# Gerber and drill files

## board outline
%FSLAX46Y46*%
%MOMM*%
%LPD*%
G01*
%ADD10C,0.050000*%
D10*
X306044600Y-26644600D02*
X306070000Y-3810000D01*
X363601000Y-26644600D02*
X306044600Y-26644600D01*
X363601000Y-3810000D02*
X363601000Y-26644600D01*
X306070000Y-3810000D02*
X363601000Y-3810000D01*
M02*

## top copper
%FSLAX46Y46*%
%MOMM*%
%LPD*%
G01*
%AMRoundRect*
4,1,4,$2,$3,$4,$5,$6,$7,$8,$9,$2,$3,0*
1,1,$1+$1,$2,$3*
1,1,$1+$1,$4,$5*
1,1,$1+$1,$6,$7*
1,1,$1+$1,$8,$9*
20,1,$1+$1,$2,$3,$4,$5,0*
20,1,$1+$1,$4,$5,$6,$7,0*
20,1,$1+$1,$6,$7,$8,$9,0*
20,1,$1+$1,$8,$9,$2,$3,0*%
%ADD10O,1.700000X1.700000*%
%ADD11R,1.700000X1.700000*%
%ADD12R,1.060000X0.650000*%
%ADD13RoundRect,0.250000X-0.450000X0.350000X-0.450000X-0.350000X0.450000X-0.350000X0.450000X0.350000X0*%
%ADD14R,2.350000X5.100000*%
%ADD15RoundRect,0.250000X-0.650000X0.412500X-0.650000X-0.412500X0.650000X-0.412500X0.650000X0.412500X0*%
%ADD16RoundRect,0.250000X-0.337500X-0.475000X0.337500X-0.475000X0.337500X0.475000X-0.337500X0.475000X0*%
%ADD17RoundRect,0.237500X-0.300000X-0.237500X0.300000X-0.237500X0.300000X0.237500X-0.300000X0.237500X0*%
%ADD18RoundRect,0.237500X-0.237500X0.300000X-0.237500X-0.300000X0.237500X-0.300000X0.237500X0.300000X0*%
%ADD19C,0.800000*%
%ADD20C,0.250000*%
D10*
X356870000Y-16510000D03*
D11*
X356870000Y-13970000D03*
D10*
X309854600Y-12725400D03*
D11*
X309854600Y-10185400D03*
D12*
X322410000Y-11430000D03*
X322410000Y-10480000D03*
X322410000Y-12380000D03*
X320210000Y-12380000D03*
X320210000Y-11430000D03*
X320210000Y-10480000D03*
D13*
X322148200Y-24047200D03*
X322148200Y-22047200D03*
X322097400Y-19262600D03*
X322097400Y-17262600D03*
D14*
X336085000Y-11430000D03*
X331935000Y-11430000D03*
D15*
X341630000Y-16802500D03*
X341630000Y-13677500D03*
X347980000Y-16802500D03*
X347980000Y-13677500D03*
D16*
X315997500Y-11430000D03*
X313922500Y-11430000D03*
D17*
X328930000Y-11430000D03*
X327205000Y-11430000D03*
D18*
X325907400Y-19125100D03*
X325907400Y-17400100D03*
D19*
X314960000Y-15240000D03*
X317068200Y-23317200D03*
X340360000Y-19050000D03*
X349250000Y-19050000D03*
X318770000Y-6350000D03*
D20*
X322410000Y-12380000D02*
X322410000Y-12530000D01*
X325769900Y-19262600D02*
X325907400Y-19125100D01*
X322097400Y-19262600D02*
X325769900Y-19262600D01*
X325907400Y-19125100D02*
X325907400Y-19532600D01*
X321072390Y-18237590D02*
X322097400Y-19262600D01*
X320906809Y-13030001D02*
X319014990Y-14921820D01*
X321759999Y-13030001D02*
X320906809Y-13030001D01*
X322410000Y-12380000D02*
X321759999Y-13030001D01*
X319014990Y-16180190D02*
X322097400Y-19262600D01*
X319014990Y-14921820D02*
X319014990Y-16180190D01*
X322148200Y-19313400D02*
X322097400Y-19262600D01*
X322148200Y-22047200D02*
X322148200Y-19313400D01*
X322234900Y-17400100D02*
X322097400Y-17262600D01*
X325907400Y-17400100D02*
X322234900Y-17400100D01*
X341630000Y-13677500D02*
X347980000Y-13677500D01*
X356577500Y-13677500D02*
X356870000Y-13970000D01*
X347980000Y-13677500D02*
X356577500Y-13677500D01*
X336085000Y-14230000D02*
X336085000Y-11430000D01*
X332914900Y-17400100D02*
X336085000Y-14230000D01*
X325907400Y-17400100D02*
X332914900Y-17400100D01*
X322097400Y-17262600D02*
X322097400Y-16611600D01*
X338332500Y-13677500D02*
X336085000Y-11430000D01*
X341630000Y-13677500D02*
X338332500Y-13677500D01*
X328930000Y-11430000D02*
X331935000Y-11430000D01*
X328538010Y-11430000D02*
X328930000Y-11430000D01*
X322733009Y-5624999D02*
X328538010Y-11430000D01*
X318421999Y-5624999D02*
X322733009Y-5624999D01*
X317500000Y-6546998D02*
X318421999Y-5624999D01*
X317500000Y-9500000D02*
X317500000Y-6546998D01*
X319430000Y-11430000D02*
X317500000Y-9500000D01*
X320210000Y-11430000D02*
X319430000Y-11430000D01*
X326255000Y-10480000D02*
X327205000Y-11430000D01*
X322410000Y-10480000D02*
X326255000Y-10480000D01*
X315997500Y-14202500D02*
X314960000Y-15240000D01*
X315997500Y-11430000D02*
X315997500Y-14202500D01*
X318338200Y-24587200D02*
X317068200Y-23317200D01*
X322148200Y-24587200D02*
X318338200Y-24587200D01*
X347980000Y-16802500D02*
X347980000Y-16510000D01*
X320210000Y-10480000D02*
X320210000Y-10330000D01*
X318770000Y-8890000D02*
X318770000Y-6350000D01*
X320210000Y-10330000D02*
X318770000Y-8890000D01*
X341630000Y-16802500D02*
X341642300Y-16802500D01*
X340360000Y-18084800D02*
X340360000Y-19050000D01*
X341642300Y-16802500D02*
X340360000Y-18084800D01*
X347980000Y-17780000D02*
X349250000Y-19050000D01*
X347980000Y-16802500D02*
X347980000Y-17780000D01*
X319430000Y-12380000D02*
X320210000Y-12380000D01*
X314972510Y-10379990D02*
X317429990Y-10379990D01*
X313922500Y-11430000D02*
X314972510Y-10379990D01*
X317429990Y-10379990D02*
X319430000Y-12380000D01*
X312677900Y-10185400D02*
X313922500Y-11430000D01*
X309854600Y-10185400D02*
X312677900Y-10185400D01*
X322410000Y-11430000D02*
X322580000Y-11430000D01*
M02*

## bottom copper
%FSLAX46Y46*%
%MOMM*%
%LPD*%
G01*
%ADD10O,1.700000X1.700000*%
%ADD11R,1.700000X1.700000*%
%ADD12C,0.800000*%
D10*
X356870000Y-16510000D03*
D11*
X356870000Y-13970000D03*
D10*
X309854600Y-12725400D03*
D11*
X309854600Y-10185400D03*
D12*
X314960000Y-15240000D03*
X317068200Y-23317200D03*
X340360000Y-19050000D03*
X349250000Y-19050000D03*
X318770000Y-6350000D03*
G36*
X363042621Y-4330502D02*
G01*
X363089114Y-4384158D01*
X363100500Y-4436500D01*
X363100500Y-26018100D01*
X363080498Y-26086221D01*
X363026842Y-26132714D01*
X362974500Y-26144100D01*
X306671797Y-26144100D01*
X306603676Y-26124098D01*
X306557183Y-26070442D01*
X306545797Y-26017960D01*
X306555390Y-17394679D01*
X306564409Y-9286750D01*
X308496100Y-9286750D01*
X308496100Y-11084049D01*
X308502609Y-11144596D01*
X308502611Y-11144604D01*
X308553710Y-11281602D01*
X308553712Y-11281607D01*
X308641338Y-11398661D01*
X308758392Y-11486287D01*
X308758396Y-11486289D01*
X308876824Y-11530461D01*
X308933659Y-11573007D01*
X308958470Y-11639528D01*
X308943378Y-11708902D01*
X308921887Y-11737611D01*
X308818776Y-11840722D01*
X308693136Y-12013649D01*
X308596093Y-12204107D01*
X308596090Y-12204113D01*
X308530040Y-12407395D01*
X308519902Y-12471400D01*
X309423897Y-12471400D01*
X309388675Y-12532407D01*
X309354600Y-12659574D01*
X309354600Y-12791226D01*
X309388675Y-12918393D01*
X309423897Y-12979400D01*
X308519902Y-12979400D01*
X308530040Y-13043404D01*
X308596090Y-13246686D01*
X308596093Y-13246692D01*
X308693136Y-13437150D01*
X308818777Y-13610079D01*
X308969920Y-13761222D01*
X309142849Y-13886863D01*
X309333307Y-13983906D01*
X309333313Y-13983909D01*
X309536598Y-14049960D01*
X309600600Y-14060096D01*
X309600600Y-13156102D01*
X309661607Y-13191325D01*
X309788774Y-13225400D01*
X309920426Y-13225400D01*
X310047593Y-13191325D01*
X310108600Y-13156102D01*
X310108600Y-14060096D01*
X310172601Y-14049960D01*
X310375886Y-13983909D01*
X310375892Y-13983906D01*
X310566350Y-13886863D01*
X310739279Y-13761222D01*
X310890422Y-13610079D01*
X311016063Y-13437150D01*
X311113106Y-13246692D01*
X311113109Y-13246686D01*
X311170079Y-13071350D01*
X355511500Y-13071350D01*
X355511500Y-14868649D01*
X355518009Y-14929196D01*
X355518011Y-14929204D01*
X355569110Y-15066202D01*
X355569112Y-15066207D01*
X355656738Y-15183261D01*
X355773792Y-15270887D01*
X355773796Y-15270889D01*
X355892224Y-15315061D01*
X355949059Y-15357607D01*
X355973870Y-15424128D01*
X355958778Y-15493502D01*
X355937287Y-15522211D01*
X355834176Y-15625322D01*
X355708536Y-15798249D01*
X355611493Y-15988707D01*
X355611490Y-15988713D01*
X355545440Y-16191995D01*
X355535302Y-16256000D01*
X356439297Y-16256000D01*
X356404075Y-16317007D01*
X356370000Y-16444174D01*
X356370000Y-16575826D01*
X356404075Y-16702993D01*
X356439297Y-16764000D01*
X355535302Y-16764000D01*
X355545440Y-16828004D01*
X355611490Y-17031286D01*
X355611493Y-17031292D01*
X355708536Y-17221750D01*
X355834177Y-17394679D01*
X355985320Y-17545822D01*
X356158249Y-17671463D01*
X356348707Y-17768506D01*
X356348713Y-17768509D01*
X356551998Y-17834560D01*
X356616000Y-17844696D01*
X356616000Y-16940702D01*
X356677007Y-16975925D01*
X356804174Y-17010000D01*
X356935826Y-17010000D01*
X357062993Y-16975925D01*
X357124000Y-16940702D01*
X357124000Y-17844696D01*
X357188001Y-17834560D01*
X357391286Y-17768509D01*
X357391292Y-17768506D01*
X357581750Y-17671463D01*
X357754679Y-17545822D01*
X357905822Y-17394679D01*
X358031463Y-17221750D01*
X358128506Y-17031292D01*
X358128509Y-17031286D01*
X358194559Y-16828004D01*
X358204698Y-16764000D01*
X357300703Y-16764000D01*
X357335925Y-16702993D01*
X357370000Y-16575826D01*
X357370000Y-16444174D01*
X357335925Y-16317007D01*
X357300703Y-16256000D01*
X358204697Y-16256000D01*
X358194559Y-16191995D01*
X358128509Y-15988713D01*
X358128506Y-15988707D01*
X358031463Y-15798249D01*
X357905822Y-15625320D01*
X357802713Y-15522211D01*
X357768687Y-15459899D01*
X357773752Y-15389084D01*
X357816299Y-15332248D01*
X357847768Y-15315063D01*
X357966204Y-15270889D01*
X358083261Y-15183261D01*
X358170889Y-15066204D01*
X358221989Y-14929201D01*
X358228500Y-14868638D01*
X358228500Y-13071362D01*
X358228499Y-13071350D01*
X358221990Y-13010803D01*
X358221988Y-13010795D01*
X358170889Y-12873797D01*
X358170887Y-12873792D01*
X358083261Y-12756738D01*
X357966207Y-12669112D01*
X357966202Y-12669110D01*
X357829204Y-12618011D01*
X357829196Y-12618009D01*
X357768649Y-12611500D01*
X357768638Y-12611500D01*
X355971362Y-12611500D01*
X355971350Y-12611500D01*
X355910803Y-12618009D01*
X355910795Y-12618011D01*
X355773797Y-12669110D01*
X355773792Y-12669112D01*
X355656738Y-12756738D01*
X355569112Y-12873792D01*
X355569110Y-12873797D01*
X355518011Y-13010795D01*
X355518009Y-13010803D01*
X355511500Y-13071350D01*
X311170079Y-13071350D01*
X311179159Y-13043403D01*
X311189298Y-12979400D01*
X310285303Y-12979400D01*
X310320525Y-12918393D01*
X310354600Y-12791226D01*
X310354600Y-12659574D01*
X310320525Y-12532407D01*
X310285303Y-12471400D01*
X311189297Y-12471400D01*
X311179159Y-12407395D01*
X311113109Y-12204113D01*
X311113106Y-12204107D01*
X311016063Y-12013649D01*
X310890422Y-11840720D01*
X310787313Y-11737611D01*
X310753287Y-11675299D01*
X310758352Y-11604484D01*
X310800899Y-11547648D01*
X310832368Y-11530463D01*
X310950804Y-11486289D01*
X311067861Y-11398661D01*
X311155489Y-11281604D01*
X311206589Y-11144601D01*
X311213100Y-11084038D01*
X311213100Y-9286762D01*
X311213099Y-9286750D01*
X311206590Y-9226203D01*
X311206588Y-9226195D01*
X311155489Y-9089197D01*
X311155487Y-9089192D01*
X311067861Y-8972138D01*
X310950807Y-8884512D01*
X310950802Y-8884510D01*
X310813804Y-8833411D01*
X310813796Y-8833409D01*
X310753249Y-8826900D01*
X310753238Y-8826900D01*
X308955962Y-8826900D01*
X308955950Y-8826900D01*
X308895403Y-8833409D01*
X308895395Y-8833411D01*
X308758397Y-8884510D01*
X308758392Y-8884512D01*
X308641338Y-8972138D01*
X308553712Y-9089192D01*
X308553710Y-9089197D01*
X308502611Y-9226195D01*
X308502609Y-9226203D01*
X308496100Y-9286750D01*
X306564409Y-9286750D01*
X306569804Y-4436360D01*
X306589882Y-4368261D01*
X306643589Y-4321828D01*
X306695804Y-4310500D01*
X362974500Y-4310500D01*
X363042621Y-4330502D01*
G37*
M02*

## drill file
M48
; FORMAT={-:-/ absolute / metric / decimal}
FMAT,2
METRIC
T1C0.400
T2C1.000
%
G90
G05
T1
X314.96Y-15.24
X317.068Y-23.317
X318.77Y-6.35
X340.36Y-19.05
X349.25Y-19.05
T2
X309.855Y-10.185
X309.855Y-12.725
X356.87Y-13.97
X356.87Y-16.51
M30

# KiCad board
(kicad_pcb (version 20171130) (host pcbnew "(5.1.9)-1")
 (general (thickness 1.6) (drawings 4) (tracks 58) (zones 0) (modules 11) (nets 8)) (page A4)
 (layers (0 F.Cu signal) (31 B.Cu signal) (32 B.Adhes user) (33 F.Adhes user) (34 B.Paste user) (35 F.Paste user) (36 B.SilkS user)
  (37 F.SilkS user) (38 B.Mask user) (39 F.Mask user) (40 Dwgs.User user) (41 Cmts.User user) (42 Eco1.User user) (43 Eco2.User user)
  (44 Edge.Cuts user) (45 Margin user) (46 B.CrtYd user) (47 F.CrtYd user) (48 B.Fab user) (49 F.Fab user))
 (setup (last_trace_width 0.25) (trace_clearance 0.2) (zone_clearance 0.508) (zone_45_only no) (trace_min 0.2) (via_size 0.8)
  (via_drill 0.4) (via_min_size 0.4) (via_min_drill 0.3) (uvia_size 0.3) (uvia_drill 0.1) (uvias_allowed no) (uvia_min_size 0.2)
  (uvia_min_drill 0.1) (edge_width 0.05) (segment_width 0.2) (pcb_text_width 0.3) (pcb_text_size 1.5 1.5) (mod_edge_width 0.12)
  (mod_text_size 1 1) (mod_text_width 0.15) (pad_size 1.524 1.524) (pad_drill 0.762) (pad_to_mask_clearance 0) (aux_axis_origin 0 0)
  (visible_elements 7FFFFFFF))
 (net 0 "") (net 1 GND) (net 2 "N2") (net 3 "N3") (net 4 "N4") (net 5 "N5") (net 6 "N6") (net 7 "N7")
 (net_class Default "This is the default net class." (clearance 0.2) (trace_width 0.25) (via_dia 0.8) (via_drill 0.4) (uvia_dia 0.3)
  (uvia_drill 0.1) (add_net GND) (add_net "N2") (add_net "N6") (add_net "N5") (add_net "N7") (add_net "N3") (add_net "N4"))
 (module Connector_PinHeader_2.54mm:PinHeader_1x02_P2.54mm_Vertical (layer F.Cu) (at 356.87 13.97)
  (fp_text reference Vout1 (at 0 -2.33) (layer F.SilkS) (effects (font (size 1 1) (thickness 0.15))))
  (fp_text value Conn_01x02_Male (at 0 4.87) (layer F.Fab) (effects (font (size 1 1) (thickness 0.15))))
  (pad 2 thru_hole oval (at 0 2.54) (size 1.7 1.7) (drill 1) (layers *.Cu *.Mask) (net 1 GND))
  (pad 1 thru_hole rect (at 0 0) (size 1.7 1.7) (drill 1) (layers *.Cu *.Mask) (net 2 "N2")))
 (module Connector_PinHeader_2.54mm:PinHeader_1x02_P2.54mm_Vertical (layer F.Cu) (at 309.8546 10.1854)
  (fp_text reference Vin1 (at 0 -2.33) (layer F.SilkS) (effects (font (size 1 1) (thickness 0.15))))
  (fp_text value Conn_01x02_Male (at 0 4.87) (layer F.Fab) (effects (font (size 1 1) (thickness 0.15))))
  (pad 2 thru_hole oval (at 0 2.54) (size 1.7 1.7) (drill 1) (layers *.Cu *.Mask) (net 1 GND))
  (pad 1 thru_hole rect (at 0 0) (size 1.7 1.7) (drill 1) (layers *.Cu *.Mask) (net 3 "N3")))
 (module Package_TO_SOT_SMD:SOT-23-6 (layer F.Cu) (at 321.31 11.43)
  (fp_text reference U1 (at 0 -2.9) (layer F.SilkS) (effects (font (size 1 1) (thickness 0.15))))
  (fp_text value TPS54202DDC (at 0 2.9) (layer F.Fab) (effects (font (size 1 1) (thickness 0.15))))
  (pad 5 smd rect (at 1.1 0) (size 1.06 0.65) (layers F.Cu F.Paste F.Mask) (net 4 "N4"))
  (pad 6 smd rect (at 1.1 -0.95) (size 1.06 0.65) (layers F.Cu F.Paste F.Mask) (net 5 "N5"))
  (pad 4 smd rect (at 1.1 0.95) (size 1.06 0.65) (layers F.Cu F.Paste F.Mask) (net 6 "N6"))
  (pad 3 smd rect (at -1.1 0.95) (size 1.06 0.65) (layers F.Cu F.Paste F.Mask) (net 3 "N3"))
  (pad 2 smd rect (at -1.1 0) (size 1.06 0.65) (layers F.Cu F.Paste F.Mask) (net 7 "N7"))
  (pad 1 smd rect (at -1.1 -0.95) (size 1.06 0.65) (layers F.Cu F.Paste F.Mask) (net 1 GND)))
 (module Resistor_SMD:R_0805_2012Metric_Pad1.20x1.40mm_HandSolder (layer F.Cu) (at 322.1482 23.0472 270)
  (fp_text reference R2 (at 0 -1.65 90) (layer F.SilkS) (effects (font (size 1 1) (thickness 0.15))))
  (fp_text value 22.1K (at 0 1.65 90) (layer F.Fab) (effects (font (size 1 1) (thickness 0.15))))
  (pad 2 smd roundrect (at 1 0 270) (size 1.2 1.4) (layers F.Cu F.Paste F.Mask) (roundrect_rratio 0.208333) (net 1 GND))
  (pad 1 smd roundrect (at -1 0 270) (size 1.2 1.4) (layers F.Cu F.Paste F.Mask) (roundrect_rratio 0.208333) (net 6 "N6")))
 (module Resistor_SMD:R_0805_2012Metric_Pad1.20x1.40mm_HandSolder (layer F.Cu) (at 322.0974 18.2626 270)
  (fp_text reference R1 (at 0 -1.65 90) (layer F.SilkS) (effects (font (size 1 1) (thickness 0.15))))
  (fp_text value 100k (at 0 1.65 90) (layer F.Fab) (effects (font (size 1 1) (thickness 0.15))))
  (pad 2 smd roundrect (at 1 0 270) (size 1.2 1.4) (layers F.Cu F.Paste F.Mask) (roundrect_rratio 0.208333) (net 6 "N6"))
  (pad 1 smd roundrect (at -1 0 270) (size 1.2 1.4) (layers F.Cu F.Paste F.Mask) (roundrect_rratio 0.208333) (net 2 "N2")))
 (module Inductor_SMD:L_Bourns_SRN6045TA (layer F.Cu) (at 334.01 11.43)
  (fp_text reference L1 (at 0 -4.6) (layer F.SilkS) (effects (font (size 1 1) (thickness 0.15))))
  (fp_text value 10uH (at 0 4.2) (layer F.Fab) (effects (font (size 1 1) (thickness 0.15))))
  (pad 2 smd rect (at 2.075 0) (size 2.35 5.1) (layers F.Cu F.Paste F.Mask) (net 2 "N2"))
  (pad 1 smd rect (at -2.075 0) (size 2.35 5.1) (layers F.Cu F.Paste F.Mask) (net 7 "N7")))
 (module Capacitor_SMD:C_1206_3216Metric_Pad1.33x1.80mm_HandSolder (layer F.Cu) (at 341.63 15.24 270)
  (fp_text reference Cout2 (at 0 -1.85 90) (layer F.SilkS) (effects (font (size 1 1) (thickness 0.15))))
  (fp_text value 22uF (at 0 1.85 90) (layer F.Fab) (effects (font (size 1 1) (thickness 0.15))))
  (pad 2 smd roundrect (at 1.5625 0 270) (size 1.325 1.8) (layers F.Cu F.Paste F.Mask) (roundrect_rratio 0.188679) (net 1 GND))
  (pad 1 smd roundrect (at -1.5625 0 270) (size 1.325 1.8) (layers F.Cu F.Paste F.Mask) (roundrect_rratio 0.188679) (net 2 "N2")))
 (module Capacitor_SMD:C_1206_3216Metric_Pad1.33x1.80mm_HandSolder (layer F.Cu) (at 347.98 15.24 270)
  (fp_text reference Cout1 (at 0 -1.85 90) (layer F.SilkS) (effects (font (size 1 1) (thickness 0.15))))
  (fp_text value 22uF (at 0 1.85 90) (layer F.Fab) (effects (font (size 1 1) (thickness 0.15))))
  (pad 2 smd roundrect (at 1.5625 0 270) (size 1.325 1.8) (layers F.Cu F.Paste F.Mask) (roundrect_rratio 0.188679) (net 1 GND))
  (pad 1 smd roundrect (at -1.5625 0 270) (size 1.325 1.8) (layers F.Cu F.Paste F.Mask) (roundrect_rratio 0.188679) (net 2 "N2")))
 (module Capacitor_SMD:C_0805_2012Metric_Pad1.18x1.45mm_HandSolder (layer F.Cu) (at 314.96 11.43)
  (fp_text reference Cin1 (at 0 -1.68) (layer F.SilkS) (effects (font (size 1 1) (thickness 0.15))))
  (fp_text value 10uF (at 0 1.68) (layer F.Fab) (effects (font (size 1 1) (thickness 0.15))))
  (pad 2 smd roundrect (at 1.0375 0) (size 1.175 1.45) (layers F.Cu F.Paste F.Mask) (roundrect_rratio 0.212766) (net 1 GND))
  (pad 1 smd roundrect (at -1.0375 0) (size 1.175 1.45) (layers F.Cu F.Paste F.Mask) (roundrect_rratio 0.212766) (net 3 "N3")))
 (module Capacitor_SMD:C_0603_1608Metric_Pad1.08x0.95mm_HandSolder (layer F.Cu) (at 328.0675 11.43)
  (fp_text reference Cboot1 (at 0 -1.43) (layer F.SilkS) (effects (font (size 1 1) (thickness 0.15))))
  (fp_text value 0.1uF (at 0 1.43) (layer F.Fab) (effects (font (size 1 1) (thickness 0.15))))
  (pad 2 smd roundrect (at 0.8625 0) (size 1.075 0.95) (layers F.Cu F.Paste F.Mask) (roundrect_rratio 0.25) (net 7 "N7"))
  (pad 1 smd roundrect (at -0.8625 0) (size 1.075 0.95) (layers F.Cu F.Paste F.Mask) (roundrect_rratio 0.25) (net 5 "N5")))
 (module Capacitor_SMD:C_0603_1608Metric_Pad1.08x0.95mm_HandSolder (layer F.Cu) (at 325.9074 18.2626 270)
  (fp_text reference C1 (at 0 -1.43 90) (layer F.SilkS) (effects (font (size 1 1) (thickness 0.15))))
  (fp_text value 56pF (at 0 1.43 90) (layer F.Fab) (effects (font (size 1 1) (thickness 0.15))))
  (pad 2 smd roundrect (at 0.8625 0 270) (size 1.075 0.95) (layers F.Cu F.Paste F.Mask) (roundrect_rratio 0.25) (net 6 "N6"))
  (pad 1 smd roundrect (at -0.8625 0 270) (size 1.075 0.95) (layers F.Cu F.Paste F.Mask) (roundrect_rratio 0.25) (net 2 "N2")))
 (gr_line (start 306.0446 26.6446) (end 306.07 3.81) (layer Edge.Cuts) (width 0.05))
 (gr_line (start 363.601 26.6446) (end 306.0446 26.6446) (layer Edge.Cuts) (width 0.05))
 (gr_line (start 363.601 3.81) (end 363.601 26.6446) (layer Edge.Cuts) (width 0.05))
 (gr_line (start 306.07 3.81) (end 363.601 3.81) (layer Edge.Cuts) (width 0.05))
 (segment (start 322.41 12.38) (end 322.41 12.53) (width 0.25) (layer F.Cu) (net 6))
 (segment (start 325.7699 19.2626) (end 325.9074 19.1251) (width 0.25) (layer F.Cu) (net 6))
 (segment (start 322.0974 19.2626) (end 325.7699 19.2626) (width 0.25) (layer F.Cu) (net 6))
 (segment (start 325.9074 19.1251) (end 325.9074 19.5326) (width 0.25) (layer F.Cu) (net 6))
 (segment (start 321.07239 18.23759) (end 322.0974 19.2626) (width 0.25) (layer F.Cu) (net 6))
 (segment (start 320.906809 13.030001) (end 319.01499 14.92182) (width 0.25) (layer F.Cu) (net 6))
 (segment (start 321.759999 13.030001) (end 320.906809 13.030001) (width 0.25) (layer F.Cu) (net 6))
 (segment (start 322.41 12.38) (end 321.759999 13.030001) (width 0.25) (layer F.Cu) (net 6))
 (segment (start 319.01499 16.18019) (end 322.0974 19.2626) (width 0.25) (layer F.Cu) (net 6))
 (segment (start 319.01499 14.92182) (end 319.01499 16.18019) (width 0.25) (layer F.Cu) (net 6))
 (segment (start 322.1482 19.3134) (end 322.0974 19.2626) (width 0.25) (layer F.Cu) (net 6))
 (segment (start 322.1482 22.0472) (end 322.1482 19.3134) (width 0.25) (layer F.Cu) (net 6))
 (segment (start 322.2349 17.4001) (end 322.0974 17.2626) (width 0.25) (layer F.Cu) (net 2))
 (segment (start 325.9074 17.4001) (end 322.2349 17.4001) (width 0.25) (layer F.Cu) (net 2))
 (segment (start 341.63 13.6775) (end 347.98 13.6775) (width 0.25) (layer F.Cu) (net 2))
 (segment (start 356.5775 13.6775) (end 356.87 13.97) (width 0.25) (layer F.Cu) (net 2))
 (segment (start 347.98 13.6775) (end 356.5775 13.6775) (width 0.25) (layer F.Cu) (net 2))
 (segment (start 336.085 14.23) (end 336.085 11.43) (width 0.25) (layer F.Cu) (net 2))
 (segment (start 332.9149 17.4001) (end 336.085 14.23) (width 0.25) (layer F.Cu) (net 2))
 (segment (start 325.9074 17.4001) (end 332.9149 17.4001) (width 0.25) (layer F.Cu) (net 2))
 (segment (start 322.0974 17.2626) (end 322.0974 16.6116) (width 0.25) (layer F.Cu) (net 2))
 (segment (start 338.3325 13.6775) (end 336.085 11.43) (width 0.25) (layer F.Cu) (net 2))
 (segment (start 341.63 13.6775) (end 338.3325 13.6775) (width 0.25) (layer F.Cu) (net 2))
 (segment (start 328.93 11.43) (end 331.935 11.43) (width 0.25) (layer F.Cu) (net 7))
 (segment (start 328.53801 11.43) (end 328.93 11.43) (width 0.25) (layer F.Cu) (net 7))
 (segment (start 322.733009 5.624999) (end 328.53801 11.43) (width 0.25) (layer F.Cu) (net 7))
 (segment (start 318.421999 5.624999) (end 322.733009 5.624999) (width 0.25) (layer F.Cu) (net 7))
 (segment (start 317.5 6.546998) (end 318.421999 5.624999) (width 0.25) (layer F.Cu) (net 7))
 (segment (start 317.5 9.5) (end 317.5 6.546998) (width 0.25) (layer F.Cu) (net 7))
 (segment (start 319.43 11.43) (end 317.5 9.5) (width 0.25) (layer F.Cu) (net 7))
 (segment (start 320.21 11.43) (end 319.43 11.43) (width 0.25) (layer F.Cu) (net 7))
 (segment (start 326.255 10.48) (end 327.205 11.43) (width 0.25) (layer F.Cu) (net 5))
 (segment (start 322.41 10.48) (end 326.255 10.48) (width 0.25) (layer F.Cu) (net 5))
 (via (at 314.96 15.24) (size 0.8) (drill 0.4) (layers F.Cu B.Cu) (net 1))
 (segment (start 315.9975 14.2025) (end 314.96 15.24) (width 0.25) (layer F.Cu) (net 1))
 (segment (start 315.9975 11.43) (end 315.9975 14.2025) (width 0.25) (layer F.Cu) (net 1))
 (segment (start 318.3382 24.5872) (end 317.0682 23.3172) (width 0.25) (layer F.Cu) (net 1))
 (via (at 317.0682 23.3172) (size 0.8) (drill 0.4) (layers F.Cu B.Cu) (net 1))
 (segment (start 322.1482 24.5872) (end 318.3382 24.5872) (width 0.25) (layer F.Cu) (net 1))
 (via (at 340.36 19.05) (size 0.8) (drill 0.4) (layers F.Cu B.Cu) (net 1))
 (segment (start 347.98 16.8025) (end 347.98 16.51) (width 0.25) (layer F.Cu) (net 1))
 (via (at 349.25 19.05) (size 0.8) (drill 0.4) (layers F.Cu B.Cu) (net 1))
 (segment (start 320.21 10.48) (end 320.21 10.33) (width 0.25) (layer F.Cu) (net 1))
 (via (at 318.77 6.35) (size 0.8) (drill 0.4) (layers F.Cu B.Cu) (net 1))
 (segment (start 318.77 8.89) (end 318.77 6.35) (width 0.25) (layer F.Cu) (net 1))
 (segment (start 320.21 10.33) (end 318.77 8.89) (width 0.25) (layer F.Cu) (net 1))
 (segment (start 341.63 16.8025) (end 341.6423 16.8025) (width 0.25) (layer F.Cu) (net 1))
 (segment (start 340.36 18.0848) (end 340.36 19.05) (width 0.25) (layer F.Cu) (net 1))
 (segment (start 341.6423 16.8025) (end 340.36 18.0848) (width 0.25) (layer F.Cu) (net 1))
 (segment (start 347.98 17.78) (end 349.25 19.05) (width 0.25) (layer F.Cu) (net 1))
 (segment (start 347.98 16.8025) (end 347.98 17.78) (width 0.25) (layer F.Cu) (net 1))
 (segment (start 319.43 12.38) (end 320.21 12.38) (width 0.25) (layer F.Cu) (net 3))
 (segment (start 314.97251 10.37999) (end 317.42999 10.37999) (width 0.25) (layer F.Cu) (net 3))
 (segment (start 313.9225 11.43) (end 314.97251 10.37999) (width 0.25) (layer F.Cu) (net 3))
 (segment (start 317.42999 10.37999) (end 319.43 12.38) (width 0.25) (layer F.Cu) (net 3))
 (segment (start 312.6779 10.1854) (end 313.9225 11.43) (width 0.25) (layer F.Cu) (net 3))
 (segment (start 309.8546 10.1854) (end 312.6779 10.1854) (width 0.25) (layer F.Cu) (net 3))
 (segment (start 322.41 11.43) (end 322.58 11.43) (width 0.25) (layer F.Cu) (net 4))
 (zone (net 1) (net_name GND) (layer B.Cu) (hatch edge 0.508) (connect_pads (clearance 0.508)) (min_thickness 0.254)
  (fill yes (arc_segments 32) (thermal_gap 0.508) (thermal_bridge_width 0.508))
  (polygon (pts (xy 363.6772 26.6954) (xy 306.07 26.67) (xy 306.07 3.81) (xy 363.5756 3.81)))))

